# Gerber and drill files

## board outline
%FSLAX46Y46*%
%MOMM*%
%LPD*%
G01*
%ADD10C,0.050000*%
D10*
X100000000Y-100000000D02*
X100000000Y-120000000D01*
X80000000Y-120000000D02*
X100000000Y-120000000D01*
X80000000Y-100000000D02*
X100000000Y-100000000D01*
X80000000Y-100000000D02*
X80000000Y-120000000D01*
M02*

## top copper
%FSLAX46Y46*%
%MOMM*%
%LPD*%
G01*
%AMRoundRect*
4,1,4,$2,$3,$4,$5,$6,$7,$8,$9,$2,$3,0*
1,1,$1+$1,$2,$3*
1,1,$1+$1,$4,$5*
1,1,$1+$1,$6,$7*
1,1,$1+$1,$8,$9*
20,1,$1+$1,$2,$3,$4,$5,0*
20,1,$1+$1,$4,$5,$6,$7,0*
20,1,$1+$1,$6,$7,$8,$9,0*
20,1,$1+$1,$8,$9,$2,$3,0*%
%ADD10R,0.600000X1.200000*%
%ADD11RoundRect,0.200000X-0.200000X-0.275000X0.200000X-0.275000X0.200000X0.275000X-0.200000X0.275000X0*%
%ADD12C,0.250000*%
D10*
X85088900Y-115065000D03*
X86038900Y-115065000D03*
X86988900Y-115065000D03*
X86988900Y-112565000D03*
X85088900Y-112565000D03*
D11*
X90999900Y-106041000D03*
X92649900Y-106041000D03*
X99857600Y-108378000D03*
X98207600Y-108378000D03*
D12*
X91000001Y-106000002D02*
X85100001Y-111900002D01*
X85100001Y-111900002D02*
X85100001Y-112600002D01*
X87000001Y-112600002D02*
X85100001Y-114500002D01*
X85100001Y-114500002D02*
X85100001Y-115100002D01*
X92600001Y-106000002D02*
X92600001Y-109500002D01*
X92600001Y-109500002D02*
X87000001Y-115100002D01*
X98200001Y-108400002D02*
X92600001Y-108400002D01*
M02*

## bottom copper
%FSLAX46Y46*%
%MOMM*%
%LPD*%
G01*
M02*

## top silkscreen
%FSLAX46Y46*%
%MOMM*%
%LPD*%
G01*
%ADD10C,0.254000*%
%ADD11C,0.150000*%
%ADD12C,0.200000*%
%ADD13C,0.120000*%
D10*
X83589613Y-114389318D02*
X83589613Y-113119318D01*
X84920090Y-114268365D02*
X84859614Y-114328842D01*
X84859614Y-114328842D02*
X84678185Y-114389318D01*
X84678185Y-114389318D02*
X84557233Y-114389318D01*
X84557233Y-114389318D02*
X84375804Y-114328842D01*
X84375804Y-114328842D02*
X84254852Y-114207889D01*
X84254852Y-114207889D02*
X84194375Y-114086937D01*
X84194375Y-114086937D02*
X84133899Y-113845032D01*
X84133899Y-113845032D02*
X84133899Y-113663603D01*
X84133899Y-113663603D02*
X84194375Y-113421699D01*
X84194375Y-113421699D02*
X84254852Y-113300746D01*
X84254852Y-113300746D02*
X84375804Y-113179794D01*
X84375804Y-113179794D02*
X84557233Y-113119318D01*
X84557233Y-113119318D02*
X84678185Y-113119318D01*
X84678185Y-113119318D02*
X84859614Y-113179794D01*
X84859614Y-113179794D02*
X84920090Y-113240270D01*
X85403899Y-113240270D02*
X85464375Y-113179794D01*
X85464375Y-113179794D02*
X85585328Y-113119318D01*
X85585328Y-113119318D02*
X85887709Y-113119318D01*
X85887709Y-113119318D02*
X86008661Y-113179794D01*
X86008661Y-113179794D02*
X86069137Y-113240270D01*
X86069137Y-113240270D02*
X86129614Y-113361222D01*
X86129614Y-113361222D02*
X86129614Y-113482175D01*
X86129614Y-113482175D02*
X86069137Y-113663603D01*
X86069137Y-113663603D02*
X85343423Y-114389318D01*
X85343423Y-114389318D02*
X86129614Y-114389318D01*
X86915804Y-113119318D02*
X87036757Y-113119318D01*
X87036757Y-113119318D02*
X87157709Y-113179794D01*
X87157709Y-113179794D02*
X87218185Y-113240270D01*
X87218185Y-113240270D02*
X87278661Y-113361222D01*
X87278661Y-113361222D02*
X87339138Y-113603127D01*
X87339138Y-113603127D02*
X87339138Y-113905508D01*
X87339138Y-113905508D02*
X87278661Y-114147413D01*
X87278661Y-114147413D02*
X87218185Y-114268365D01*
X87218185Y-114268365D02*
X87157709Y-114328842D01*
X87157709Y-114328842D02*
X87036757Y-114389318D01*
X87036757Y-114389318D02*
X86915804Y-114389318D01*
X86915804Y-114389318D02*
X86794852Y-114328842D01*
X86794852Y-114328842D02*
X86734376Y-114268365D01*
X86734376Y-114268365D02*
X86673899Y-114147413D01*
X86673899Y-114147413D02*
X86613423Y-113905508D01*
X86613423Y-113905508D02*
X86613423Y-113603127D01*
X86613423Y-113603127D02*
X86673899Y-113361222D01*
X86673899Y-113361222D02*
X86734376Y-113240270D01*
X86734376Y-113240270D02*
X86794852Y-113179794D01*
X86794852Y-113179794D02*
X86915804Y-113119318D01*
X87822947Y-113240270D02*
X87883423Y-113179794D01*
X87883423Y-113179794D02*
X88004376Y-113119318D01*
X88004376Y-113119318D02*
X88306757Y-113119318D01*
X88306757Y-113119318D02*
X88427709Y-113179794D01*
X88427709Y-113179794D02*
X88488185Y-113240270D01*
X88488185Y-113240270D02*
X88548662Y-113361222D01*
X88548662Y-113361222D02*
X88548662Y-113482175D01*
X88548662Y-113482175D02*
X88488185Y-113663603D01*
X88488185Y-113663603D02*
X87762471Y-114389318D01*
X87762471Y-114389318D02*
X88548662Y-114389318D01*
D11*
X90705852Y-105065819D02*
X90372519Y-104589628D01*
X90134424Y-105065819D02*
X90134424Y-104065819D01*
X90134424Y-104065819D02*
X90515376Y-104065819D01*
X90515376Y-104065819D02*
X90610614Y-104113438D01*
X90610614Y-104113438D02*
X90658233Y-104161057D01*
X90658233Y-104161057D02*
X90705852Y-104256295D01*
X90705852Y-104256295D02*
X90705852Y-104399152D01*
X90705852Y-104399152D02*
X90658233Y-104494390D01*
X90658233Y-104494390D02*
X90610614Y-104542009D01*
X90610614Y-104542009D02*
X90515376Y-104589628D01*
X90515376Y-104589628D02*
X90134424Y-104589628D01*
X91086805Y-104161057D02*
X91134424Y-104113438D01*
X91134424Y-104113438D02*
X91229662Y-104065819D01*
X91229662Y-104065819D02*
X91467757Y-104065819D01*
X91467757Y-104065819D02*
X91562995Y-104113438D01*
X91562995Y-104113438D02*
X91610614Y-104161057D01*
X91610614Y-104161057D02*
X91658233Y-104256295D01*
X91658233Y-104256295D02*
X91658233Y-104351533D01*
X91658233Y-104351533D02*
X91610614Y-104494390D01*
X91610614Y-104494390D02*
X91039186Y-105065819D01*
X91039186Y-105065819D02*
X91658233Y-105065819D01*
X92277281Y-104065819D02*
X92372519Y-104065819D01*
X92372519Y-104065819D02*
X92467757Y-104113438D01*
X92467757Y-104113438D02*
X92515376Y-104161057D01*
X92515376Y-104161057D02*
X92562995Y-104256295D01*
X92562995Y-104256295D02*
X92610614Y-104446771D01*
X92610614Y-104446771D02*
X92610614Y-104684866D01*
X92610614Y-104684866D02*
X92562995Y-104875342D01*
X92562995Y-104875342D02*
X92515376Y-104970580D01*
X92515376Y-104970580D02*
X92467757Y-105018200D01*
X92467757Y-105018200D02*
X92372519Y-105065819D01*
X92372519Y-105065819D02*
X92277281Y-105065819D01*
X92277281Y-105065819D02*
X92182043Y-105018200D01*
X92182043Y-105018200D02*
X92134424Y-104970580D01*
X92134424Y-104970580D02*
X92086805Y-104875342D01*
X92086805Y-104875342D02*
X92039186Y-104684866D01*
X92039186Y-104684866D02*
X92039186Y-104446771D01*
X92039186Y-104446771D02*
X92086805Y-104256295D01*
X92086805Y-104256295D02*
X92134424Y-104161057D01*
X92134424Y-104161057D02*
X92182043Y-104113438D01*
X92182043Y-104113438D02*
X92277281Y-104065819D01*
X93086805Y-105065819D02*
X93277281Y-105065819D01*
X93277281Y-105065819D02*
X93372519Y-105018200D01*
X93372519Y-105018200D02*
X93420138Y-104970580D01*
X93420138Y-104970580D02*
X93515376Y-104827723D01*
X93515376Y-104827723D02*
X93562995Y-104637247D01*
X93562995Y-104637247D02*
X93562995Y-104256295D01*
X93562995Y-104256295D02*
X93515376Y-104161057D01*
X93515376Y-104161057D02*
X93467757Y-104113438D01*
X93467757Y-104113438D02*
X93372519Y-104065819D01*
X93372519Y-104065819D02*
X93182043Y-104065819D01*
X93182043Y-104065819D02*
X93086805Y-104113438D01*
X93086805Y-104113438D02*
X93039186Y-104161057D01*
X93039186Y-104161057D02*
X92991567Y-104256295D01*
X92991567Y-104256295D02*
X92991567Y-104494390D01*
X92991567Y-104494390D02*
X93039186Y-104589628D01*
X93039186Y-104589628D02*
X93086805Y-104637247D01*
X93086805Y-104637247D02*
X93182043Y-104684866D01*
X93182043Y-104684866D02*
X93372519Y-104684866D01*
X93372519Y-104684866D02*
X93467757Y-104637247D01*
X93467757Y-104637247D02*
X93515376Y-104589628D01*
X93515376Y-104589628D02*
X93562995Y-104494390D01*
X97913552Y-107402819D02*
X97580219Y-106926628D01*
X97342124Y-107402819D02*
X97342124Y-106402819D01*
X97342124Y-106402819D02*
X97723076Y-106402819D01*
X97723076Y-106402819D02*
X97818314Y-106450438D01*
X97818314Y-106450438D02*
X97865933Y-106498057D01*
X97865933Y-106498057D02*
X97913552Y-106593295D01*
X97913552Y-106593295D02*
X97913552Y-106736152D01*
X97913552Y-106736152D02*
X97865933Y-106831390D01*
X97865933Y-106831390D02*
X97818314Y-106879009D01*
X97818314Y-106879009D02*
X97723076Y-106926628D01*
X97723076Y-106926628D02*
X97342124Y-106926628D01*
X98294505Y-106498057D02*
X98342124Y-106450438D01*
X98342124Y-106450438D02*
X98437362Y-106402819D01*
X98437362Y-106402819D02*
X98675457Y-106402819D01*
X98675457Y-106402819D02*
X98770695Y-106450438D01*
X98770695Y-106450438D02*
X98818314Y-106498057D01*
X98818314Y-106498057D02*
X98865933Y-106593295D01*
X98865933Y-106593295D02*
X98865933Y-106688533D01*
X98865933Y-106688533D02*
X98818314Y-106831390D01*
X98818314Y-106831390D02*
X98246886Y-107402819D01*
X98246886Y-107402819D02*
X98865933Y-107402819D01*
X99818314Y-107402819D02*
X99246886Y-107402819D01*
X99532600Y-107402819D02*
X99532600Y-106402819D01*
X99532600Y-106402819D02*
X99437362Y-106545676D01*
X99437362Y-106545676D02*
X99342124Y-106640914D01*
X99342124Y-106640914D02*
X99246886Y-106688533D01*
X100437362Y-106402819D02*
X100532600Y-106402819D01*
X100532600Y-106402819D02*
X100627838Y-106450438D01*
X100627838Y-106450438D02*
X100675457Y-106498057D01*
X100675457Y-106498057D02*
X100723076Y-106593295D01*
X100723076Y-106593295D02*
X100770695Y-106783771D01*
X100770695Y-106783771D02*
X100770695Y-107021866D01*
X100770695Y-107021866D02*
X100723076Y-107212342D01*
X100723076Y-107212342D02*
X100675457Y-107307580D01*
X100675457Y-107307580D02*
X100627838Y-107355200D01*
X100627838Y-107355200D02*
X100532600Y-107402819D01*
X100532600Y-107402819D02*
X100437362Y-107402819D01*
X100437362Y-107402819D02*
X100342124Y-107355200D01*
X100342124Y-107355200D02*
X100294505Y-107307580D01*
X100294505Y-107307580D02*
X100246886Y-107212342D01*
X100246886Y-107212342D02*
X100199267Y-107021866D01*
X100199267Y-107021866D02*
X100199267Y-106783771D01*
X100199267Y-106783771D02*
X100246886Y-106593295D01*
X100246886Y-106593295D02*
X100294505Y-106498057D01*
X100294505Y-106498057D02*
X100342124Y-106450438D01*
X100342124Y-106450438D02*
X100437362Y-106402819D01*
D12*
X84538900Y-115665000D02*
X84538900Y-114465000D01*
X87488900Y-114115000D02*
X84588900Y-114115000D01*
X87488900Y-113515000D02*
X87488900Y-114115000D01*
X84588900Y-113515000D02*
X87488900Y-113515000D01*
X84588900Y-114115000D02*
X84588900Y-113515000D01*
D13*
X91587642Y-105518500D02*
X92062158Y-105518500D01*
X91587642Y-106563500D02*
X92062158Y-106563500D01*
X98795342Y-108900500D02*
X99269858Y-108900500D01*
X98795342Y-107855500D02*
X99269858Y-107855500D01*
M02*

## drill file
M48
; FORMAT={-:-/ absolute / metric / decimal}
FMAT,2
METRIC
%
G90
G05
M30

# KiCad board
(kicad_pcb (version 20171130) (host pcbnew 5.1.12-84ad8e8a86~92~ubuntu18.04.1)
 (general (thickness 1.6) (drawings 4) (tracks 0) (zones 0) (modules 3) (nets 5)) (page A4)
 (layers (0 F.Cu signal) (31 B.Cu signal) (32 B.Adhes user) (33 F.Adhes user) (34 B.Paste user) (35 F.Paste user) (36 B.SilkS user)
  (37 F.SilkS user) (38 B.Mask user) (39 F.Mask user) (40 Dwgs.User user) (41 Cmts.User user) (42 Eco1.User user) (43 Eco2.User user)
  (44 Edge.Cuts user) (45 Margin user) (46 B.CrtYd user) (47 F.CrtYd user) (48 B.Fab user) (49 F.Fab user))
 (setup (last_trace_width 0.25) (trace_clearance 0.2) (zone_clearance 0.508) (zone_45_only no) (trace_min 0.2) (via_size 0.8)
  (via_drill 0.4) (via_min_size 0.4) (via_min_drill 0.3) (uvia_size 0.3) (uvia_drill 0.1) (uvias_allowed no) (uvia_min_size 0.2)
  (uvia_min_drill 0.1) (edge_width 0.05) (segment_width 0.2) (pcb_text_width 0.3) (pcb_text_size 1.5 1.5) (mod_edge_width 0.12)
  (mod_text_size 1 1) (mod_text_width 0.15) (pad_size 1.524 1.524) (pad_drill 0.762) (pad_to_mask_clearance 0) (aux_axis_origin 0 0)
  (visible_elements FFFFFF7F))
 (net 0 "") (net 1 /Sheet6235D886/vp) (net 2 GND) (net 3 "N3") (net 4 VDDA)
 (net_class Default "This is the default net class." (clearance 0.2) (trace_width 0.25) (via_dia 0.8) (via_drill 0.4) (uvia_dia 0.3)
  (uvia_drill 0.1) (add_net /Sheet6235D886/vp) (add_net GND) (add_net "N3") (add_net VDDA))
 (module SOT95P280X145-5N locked (layer F.Cu) (at 86.038900 113.815000 90.000000)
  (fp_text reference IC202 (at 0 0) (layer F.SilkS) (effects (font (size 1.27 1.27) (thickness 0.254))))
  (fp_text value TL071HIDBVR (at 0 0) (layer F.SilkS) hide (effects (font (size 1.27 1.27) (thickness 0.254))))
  (fp_line (start -1.85 -1.5) (end -0.65 -1.5) (layer F.SilkS) (width 0.2))
  (fp_line (start -0.3 1.45) (end -0.3 -1.45) (layer F.SilkS) (width 0.2))
  (fp_line (start 0.3 1.45) (end -0.3 1.45) (layer F.SilkS) (width 0.2))
  (fp_line (start 0.3 -1.45) (end 0.3 1.45) (layer F.SilkS) (width 0.2))
  (fp_line (start -0.3 -1.45) (end 0.3 -1.45) (layer F.SilkS) (width 0.2))
  (pad 1 smd rect (at -1.25 -0.95 180.000000) (size 0.6 1.2) (layers F.Cu F.Mask F.Paste) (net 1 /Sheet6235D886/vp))
  (pad 2 smd rect (at -1.25 0 180.000000) (size 0.6 1.2) (layers F.Cu F.Mask F.Paste) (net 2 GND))
  (pad 3 smd rect (at -1.25 0.95 180.000000) (size 0.6 1.2) (layers F.Cu F.Mask F.Paste) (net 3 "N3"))
  (pad 4 smd rect (at 1.25 0.95 180.000000) (size 0.6 1.2) (layers F.Cu F.Mask F.Paste) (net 1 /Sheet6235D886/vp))
  (pad 5 smd rect (at 1.25 -0.95 180.000000) (size 0.6 1.2) (layers F.Cu F.Mask F.Paste) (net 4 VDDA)))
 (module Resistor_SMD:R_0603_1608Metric (layer F.Cu) (at 91.824900 106.041000)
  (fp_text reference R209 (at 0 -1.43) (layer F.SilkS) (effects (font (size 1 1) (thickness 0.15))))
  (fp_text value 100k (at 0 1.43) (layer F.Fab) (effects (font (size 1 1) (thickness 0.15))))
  (fp_line (start -0.237258 -0.5225) (end 0.237258 -0.5225) (layer F.SilkS) (width 0.12))
  (fp_line (start -0.237258 0.5225) (end 0.237258 0.5225) (layer F.SilkS) (width 0.12))
  (pad 1 smd roundrect (at -0.825 0) (size 0.8 0.95) (layers F.Cu F.Mask F.Paste) (roundrect_rratio 0.25) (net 4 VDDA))
  (pad 2 smd roundrect (at 0.825 0) (size 0.8 0.95) (layers F.Cu F.Mask F.Paste) (roundrect_rratio 0.25) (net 3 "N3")))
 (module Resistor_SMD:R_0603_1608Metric (layer F.Cu) (at 99.032600 108.378000)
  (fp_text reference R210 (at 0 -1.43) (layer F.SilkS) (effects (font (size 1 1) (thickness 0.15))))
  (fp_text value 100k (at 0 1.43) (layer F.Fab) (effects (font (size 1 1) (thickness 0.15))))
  (fp_line (start -0.237258 0.5225) (end 0.237258 0.5225) (layer F.SilkS) (width 0.12))
  (fp_line (start -0.237258 -0.5225) (end 0.237258 -0.5225) (layer F.SilkS) (width 0.12))
  (pad 2 smd roundrect (at 0.825 0) (size 0.8 0.95) (layers F.Cu F.Mask F.Paste) (roundrect_rratio 0.25) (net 2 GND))
  (pad 1 smd roundrect (at -0.825 0) (size 0.8 0.95) (layers F.Cu F.Mask F.Paste) (roundrect_rratio 0.25) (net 3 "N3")))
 (gr_line (start 100 100) (end 100 120) (layer Edge.Cuts) (width 0.05))
 (gr_line (start 80 120) (end 100 120) (layer Edge.Cuts) (width 0.05))
 (gr_line (start 80 100) (end 100 100) (layer Edge.Cuts) (width 0.05))
 (gr_line (start 80 100) (end 80 120) (layer Edge.Cuts) (width 0.05))
 (segment (start 91.000001 106.000002) (end 85.100001 111.900002) (width 0.250000) (layer F.Cu) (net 4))
 (segment (start 85.100001 111.900002) (end 85.100001 112.600002) (width 0.250000) (layer F.Cu) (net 4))
 (segment (start 87.000001 112.600002) (end 85.100001 114.500002) (width 0.250000) (layer F.Cu) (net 1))
 (segment (start 85.100001 114.500002) (end 85.100001 115.100002) (width 0.250000) (layer F.Cu) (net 1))
 (segment (start 92.600001 106.000002) (end 92.600001 109.500002) (width 0.250000) (layer F.Cu) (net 3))
 (segment (start 92.600001 109.500002) (end 87.000001 115.100002) (width 0.250000) (layer F.Cu) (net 3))
 (segment (start 98.200001 108.400002) (end 92.600001 108.400002) (width 0.250000) (layer F.Cu) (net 3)))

